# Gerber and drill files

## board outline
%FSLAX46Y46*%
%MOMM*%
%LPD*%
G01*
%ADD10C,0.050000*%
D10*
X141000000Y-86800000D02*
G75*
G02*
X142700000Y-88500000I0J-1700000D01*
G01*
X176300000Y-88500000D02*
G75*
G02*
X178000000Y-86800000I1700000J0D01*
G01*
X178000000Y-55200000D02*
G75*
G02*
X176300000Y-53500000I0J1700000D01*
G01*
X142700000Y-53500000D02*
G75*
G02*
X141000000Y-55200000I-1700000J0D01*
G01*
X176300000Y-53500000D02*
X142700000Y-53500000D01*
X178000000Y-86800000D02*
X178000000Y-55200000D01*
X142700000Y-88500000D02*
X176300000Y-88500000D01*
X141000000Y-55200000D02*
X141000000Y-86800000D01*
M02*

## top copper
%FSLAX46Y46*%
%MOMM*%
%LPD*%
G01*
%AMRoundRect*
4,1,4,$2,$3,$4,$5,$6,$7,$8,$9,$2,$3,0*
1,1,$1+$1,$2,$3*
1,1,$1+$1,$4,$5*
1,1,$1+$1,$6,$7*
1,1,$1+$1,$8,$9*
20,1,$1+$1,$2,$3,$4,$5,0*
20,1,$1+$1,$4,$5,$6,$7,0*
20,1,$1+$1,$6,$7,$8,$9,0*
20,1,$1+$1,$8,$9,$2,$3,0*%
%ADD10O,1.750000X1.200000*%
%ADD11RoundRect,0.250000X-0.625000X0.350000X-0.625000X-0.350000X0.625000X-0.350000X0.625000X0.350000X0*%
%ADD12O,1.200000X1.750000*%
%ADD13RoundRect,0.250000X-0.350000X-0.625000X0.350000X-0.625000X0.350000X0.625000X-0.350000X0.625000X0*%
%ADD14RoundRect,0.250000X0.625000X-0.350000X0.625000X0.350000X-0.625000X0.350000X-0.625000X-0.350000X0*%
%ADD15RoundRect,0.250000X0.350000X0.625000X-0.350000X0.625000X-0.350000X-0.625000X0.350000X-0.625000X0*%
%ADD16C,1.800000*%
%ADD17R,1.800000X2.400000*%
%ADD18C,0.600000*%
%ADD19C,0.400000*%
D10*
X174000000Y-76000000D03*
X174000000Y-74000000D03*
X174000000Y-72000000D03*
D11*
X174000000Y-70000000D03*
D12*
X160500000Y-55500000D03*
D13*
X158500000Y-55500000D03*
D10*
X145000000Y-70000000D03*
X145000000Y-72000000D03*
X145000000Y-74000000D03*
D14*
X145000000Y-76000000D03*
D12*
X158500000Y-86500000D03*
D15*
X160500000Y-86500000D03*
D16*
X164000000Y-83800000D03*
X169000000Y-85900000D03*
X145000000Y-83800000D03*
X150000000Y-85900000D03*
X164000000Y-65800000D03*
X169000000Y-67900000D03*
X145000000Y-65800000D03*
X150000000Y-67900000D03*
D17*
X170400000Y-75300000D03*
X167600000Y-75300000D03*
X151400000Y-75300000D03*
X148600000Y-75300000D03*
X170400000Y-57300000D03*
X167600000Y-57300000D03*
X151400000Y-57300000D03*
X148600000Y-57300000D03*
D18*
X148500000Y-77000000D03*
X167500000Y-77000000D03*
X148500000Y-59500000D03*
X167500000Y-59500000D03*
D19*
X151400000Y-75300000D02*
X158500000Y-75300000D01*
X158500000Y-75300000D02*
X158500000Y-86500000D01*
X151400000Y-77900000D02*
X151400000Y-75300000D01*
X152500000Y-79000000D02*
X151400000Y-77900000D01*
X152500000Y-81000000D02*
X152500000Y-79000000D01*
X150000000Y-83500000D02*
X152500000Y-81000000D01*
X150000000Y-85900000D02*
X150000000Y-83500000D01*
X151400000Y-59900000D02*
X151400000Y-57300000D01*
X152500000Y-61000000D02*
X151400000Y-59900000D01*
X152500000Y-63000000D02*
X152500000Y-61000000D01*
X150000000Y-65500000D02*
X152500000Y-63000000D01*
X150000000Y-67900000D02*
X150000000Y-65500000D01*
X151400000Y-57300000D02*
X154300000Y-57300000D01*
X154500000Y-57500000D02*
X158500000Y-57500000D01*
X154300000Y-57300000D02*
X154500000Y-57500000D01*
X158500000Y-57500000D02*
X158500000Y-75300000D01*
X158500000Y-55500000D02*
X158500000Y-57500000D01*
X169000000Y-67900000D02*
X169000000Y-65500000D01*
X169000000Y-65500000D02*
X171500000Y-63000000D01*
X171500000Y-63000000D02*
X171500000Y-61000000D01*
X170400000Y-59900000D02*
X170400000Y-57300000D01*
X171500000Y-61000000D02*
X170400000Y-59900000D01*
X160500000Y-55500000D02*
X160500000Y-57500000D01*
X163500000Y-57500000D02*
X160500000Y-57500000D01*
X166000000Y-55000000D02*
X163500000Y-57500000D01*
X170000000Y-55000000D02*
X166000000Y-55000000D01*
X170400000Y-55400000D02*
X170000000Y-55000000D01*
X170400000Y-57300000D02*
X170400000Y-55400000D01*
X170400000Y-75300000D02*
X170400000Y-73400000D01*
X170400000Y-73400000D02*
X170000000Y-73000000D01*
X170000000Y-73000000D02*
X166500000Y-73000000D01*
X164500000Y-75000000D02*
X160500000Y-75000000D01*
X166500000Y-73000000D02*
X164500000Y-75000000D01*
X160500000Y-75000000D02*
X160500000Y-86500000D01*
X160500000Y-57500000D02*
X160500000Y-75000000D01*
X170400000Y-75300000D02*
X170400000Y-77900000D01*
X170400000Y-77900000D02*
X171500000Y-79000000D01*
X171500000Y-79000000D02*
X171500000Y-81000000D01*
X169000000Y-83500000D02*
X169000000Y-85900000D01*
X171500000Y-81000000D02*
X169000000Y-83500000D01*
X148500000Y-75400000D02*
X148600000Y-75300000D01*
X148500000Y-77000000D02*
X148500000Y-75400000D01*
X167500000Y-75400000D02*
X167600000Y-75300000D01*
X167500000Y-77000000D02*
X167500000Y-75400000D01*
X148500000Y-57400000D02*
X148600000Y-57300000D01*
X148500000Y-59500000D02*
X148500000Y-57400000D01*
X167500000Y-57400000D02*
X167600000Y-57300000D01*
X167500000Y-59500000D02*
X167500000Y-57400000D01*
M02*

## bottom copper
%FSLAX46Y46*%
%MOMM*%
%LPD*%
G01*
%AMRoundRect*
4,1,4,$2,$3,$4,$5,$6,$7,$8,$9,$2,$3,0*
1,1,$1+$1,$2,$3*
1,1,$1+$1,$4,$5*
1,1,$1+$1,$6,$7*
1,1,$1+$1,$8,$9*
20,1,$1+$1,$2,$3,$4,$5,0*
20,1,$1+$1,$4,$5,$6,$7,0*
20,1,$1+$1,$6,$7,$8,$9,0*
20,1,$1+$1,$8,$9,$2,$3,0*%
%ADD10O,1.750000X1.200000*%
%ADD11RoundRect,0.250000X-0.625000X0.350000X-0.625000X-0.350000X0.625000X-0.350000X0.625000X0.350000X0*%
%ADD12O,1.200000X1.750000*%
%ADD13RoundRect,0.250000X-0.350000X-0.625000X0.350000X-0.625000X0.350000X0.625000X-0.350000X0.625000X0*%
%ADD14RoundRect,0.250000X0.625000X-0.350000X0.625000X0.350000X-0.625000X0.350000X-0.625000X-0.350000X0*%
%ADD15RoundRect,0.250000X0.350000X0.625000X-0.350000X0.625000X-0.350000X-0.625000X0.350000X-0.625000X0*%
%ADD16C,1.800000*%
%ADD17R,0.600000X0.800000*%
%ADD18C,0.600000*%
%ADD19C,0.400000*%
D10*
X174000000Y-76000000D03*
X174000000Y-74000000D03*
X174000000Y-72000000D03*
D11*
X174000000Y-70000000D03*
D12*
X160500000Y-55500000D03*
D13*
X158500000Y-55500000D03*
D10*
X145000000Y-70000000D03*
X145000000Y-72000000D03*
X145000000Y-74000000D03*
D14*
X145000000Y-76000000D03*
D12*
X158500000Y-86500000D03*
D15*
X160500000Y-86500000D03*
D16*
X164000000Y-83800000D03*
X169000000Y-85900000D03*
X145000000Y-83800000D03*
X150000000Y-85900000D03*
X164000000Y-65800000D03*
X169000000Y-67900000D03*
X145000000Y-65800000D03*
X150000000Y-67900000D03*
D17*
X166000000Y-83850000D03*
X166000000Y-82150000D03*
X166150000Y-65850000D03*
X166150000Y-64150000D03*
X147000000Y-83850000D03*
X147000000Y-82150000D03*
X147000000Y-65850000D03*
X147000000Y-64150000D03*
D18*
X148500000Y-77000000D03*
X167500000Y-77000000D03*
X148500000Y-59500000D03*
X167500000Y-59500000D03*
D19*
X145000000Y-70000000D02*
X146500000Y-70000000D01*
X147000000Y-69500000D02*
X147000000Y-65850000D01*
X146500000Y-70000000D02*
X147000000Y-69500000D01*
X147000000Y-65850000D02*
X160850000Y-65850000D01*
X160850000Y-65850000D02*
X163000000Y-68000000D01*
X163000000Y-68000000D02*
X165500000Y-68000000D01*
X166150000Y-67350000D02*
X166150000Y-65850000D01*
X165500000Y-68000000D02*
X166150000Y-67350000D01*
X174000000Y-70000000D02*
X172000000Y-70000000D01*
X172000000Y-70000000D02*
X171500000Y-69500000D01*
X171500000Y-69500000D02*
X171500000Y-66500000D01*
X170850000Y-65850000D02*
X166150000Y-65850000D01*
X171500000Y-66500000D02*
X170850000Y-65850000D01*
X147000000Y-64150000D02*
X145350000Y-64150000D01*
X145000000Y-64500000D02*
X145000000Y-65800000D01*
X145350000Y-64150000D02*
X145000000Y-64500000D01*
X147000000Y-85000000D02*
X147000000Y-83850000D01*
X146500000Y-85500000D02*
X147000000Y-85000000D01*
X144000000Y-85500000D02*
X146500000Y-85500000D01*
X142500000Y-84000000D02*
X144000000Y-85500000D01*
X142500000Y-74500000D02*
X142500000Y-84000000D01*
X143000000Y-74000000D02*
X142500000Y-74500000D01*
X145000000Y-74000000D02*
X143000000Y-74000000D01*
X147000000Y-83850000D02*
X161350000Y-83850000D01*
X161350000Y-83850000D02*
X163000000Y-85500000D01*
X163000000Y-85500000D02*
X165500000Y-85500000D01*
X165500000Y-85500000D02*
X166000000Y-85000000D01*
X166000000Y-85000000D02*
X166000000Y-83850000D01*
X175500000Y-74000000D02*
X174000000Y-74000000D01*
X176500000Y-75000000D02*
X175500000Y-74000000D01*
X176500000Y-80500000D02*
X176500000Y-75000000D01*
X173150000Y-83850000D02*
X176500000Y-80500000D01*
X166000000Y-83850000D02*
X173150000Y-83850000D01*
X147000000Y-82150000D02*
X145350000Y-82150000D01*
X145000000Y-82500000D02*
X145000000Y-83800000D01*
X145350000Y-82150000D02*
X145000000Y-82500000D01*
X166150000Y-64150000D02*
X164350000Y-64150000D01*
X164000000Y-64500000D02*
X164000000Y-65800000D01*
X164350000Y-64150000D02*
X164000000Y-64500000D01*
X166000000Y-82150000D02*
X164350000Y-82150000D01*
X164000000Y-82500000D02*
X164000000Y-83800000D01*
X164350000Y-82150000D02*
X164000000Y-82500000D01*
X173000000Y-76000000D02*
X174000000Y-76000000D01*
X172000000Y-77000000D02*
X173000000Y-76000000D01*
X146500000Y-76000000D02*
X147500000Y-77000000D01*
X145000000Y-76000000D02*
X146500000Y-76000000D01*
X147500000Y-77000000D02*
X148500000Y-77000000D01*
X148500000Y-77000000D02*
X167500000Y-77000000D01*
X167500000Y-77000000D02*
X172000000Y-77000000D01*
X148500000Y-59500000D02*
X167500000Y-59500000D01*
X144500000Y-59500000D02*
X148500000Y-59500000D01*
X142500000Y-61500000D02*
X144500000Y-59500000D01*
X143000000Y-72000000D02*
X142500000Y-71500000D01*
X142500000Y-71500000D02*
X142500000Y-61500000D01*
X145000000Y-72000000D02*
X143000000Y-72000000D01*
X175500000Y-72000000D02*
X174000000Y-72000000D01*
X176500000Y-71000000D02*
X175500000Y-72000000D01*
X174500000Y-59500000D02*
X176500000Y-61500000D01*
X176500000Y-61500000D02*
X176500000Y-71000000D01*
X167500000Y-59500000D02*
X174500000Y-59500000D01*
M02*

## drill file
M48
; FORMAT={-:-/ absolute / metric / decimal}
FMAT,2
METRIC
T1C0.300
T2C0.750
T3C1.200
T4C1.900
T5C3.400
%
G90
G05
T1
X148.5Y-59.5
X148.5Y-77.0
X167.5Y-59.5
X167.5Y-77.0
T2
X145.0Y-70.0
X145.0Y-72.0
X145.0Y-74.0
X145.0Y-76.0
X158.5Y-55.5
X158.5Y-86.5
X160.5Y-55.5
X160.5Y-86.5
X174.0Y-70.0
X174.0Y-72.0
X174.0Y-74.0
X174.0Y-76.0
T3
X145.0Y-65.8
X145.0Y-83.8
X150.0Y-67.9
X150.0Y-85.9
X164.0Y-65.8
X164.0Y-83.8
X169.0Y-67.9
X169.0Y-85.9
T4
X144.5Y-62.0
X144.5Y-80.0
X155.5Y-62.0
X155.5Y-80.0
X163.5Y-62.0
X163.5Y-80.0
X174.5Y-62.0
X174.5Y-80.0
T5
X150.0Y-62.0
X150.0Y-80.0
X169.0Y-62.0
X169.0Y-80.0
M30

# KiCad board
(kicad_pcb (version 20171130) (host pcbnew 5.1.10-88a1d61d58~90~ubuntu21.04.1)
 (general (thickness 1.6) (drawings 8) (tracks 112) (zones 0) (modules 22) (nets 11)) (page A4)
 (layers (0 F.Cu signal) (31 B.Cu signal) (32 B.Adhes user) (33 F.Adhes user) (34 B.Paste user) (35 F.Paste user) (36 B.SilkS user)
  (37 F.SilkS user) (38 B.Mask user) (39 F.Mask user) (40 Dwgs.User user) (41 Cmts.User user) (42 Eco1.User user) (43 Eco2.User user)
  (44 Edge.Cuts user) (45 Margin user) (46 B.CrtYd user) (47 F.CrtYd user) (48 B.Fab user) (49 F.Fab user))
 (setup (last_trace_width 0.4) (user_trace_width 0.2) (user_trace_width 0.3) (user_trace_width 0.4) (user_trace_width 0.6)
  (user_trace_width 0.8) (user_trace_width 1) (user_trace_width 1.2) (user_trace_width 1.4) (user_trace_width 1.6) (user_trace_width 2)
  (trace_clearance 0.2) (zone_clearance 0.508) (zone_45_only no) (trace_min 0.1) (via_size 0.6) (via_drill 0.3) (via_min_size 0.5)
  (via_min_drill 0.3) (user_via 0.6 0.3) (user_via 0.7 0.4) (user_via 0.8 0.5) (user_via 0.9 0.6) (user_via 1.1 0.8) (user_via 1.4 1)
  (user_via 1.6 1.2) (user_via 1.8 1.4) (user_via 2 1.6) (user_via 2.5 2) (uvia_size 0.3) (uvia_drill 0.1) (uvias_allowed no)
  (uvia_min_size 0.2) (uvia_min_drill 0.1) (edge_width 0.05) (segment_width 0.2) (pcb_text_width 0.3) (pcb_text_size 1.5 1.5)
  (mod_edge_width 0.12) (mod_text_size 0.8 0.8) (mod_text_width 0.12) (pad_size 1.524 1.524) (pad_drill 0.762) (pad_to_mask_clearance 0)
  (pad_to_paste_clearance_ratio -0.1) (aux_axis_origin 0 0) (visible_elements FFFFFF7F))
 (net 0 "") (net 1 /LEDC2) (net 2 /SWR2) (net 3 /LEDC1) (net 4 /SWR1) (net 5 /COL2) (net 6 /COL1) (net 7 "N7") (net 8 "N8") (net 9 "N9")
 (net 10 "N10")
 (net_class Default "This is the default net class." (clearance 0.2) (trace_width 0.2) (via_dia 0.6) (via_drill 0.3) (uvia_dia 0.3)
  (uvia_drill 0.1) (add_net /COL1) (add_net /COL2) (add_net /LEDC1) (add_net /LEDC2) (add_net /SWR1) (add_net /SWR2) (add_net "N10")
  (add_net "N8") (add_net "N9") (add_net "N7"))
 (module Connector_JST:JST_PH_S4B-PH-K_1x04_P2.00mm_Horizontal (layer B.Cu) (at 174 70 270)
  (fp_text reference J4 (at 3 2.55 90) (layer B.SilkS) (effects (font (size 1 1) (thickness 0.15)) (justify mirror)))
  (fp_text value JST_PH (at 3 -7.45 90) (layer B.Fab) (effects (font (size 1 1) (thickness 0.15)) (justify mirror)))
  (pad 4 thru_hole oval (at 6 0 270) (size 1.2 1.75) (drill 0.75) (layers *.Cu *.Mask) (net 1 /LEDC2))
  (pad 3 thru_hole oval (at 4 0 270) (size 1.2 1.75) (drill 0.75) (layers *.Cu *.Mask) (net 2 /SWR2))
  (pad 2 thru_hole oval (at 2 0 270) (size 1.2 1.75) (drill 0.75) (layers *.Cu *.Mask) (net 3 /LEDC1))
  (pad 1 thru_hole roundrect (at 0 0 270) (size 1.2 1.75) (drill 0.75) (layers *.Cu *.Mask) (roundrect_rratio 0.208333) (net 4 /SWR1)))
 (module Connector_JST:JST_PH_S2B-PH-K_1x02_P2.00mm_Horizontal (layer B.Cu) (at 158.5 55.5)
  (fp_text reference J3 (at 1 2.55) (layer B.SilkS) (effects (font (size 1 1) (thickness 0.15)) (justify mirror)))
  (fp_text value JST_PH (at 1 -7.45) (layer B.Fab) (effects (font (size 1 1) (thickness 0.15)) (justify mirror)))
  (pad 2 thru_hole oval (at 2 0) (size 1.2 1.75) (drill 0.75) (layers *.Cu *.Mask) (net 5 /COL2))
  (pad 1 thru_hole roundrect (at 0 0) (size 1.2 1.75) (drill 0.75) (layers *.Cu *.Mask) (roundrect_rratio 0.208333) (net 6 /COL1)))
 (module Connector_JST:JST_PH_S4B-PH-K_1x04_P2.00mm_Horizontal (layer B.Cu) (at 145 76 90)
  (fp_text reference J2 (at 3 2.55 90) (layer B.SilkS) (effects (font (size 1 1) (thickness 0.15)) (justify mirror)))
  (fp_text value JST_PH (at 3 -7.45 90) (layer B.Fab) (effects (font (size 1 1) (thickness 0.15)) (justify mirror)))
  (pad 4 thru_hole oval (at 6 0 90) (size 1.2 1.75) (drill 0.75) (layers *.Cu *.Mask) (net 4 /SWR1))
  (pad 3 thru_hole oval (at 4 0 90) (size 1.2 1.75) (drill 0.75) (layers *.Cu *.Mask) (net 3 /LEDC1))
  (pad 2 thru_hole oval (at 2 0 90) (size 1.2 1.75) (drill 0.75) (layers *.Cu *.Mask) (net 2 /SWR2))
  (pad 1 thru_hole roundrect (at 0 0 90) (size 1.2 1.75) (drill 0.75) (layers *.Cu *.Mask) (roundrect_rratio 0.208333) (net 1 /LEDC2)))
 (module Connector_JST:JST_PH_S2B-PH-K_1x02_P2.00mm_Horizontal (layer B.Cu) (at 160.5 86.5 180)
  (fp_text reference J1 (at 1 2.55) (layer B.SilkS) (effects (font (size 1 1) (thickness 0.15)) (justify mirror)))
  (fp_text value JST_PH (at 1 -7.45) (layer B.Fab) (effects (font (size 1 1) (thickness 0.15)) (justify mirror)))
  (pad 2 thru_hole oval (at 2 0 180) (size 1.2 1.75) (drill 0.75) (layers *.Cu *.Mask) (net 6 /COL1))
  (pad 1 thru_hole roundrect (at 0 0 180) (size 1.2 1.75) (drill 0.75) (layers *.Cu *.Mask) (roundrect_rratio 0.208333) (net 5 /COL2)))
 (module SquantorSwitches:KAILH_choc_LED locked (layer F.Cu) (at 169 80 180)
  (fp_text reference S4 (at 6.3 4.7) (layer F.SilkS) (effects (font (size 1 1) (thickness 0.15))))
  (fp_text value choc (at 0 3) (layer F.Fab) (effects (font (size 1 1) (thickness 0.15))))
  (pad 2 thru_hole circle (at 5 -3.8 180) (size 1.8 1.8) (drill 1.2) (layers *.Cu *.Mask) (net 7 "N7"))
  (pad 1 thru_hole circle (at 0 -5.9 180) (size 1.8 1.8) (drill 1.2) (layers *.Cu *.Mask) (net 5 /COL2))
  (pad "" np_thru_hole circle (at 5.5 0 180) (size 1.9 1.9) (drill 1.9) (layers *.Cu *.Mask))
  (pad "" np_thru_hole circle (at -5.5 0 180) (size 1.9 1.9) (drill 1.9) (layers *.Cu *.Mask))
  (pad "" np_thru_hole circle (at 0 0 180) (size 3.4 3.4) (drill 3.4) (layers *.Cu *.Mask)))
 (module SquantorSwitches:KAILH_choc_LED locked (layer F.Cu) (at 150 80 180)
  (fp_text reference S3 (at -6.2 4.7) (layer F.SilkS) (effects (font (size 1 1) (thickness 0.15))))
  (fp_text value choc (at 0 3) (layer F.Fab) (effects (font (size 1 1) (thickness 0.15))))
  (pad 2 thru_hole circle (at 5 -3.8 180) (size 1.8 1.8) (drill 1.2) (layers *.Cu *.Mask) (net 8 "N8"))
  (pad 1 thru_hole circle (at 0 -5.9 180) (size 1.8 1.8) (drill 1.2) (layers *.Cu *.Mask) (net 6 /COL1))
  (pad "" np_thru_hole circle (at 5.5 0 180) (size 1.9 1.9) (drill 1.9) (layers *.Cu *.Mask))
  (pad "" np_thru_hole circle (at -5.5 0 180) (size 1.9 1.9) (drill 1.9) (layers *.Cu *.Mask))
  (pad "" np_thru_hole circle (at 0 0 180) (size 3.4 3.4) (drill 3.4) (layers *.Cu *.Mask)))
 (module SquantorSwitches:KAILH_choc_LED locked (layer F.Cu) (at 169 62 180)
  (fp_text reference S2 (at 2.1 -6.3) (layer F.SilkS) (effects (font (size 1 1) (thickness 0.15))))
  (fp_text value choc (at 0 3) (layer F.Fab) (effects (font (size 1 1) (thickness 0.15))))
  (pad 2 thru_hole circle (at 5 -3.8 180) (size 1.8 1.8) (drill 1.2) (layers *.Cu *.Mask) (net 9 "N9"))
  (pad 1 thru_hole circle (at 0 -5.9 180) (size 1.8 1.8) (drill 1.2) (layers *.Cu *.Mask) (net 5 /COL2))
  (pad "" np_thru_hole circle (at 5.5 0 180) (size 1.9 1.9) (drill 1.9) (layers *.Cu *.Mask))
  (pad "" np_thru_hole circle (at -5.5 0 180) (size 1.9 1.9) (drill 1.9) (layers *.Cu *.Mask))
  (pad "" np_thru_hole circle (at 0 0 180) (size 3.4 3.4) (drill 3.4) (layers *.Cu *.Mask)))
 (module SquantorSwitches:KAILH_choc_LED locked (layer F.Cu) (at 150 62 180)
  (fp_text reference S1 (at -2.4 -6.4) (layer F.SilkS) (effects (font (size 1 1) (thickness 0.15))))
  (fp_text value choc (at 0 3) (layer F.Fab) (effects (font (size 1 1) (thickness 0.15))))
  (pad 2 thru_hole circle (at 5 -3.8 180) (size 1.8 1.8) (drill 1.2) (layers *.Cu *.Mask) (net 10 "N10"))
  (pad 1 thru_hole circle (at 0 -5.9 180) (size 1.8 1.8) (drill 1.2) (layers *.Cu *.Mask) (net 6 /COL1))
  (pad "" np_thru_hole circle (at 5.5 0 180) (size 1.9 1.9) (drill 1.9) (layers *.Cu *.Mask))
  (pad "" np_thru_hole circle (at -5.5 0 180) (size 1.9 1.9) (drill 1.9) (layers *.Cu *.Mask))
  (pad "" np_thru_hole circle (at 0 0 180) (size 3.4 3.4) (drill 3.4) (layers *.Cu *.Mask)))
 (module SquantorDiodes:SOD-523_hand (layer B.Cu) (at 166 83 90)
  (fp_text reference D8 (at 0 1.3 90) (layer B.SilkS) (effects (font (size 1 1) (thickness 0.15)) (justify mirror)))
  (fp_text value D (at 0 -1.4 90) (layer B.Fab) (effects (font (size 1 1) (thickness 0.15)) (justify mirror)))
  (pad 1 smd rect (at -0.85 0 90) (size 0.8 0.6) (layers B.Cu B.Paste B.Mask) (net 2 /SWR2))
  (pad 2 smd rect (at 0.85 0 90) (size 0.8 0.6) (layers B.Cu B.Paste B.Mask) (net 7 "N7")))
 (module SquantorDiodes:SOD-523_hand (layer B.Cu) (at 166.15 65 90)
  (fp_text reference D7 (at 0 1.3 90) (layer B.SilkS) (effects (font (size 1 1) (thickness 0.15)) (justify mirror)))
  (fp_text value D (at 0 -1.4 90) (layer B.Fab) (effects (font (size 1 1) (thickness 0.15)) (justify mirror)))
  (pad 1 smd rect (at -0.85 0 90) (size 0.8 0.6) (layers B.Cu B.Paste B.Mask) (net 4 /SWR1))
  (pad 2 smd rect (at 0.85 0 90) (size 0.8 0.6) (layers B.Cu B.Paste B.Mask) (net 9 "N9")))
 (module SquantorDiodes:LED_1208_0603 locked (layer F.Cu) (at 169 75.3)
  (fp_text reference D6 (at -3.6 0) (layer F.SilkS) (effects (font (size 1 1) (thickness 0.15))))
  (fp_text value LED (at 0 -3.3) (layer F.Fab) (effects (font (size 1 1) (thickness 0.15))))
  (pad 2 smd rect (at 1.4 0) (size 1.8 2.4) (layers F.Cu F.Paste F.Mask) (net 5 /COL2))
  (pad 1 smd rect (at -1.4 0) (size 1.8 2.4) (layers F.Cu F.Paste F.Mask) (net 1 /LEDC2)))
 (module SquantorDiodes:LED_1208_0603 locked (layer F.Cu) (at 150 75.3)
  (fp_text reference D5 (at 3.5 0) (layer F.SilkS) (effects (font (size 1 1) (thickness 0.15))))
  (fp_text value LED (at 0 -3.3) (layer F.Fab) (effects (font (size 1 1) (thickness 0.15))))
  (pad 2 smd rect (at 1.4 0) (size 1.8 2.4) (layers F.Cu F.Paste F.Mask) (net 6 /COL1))
  (pad 1 smd rect (at -1.4 0) (size 1.8 2.4) (layers F.Cu F.Paste F.Mask) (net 1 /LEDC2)))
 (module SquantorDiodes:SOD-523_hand (layer B.Cu) (at 147 83 90)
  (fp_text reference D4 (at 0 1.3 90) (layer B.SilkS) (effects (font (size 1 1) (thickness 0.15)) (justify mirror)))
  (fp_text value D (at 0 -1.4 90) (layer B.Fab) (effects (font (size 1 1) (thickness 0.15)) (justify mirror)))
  (pad 1 smd rect (at -0.85 0 90) (size 0.8 0.6) (layers B.Cu B.Paste B.Mask) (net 2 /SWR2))
  (pad 2 smd rect (at 0.85 0 90) (size 0.8 0.6) (layers B.Cu B.Paste B.Mask) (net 8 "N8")))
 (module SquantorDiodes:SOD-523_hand (layer B.Cu) (at 147 65 90)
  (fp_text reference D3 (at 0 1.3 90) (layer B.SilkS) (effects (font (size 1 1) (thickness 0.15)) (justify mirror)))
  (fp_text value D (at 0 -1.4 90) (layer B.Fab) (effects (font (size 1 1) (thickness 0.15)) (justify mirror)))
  (pad 1 smd rect (at -0.85 0 90) (size 0.8 0.6) (layers B.Cu B.Paste B.Mask) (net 4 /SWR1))
  (pad 2 smd rect (at 0.85 0 90) (size 0.8 0.6) (layers B.Cu B.Paste B.Mask) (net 10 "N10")))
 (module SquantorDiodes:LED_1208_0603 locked (layer F.Cu) (at 169 57.3)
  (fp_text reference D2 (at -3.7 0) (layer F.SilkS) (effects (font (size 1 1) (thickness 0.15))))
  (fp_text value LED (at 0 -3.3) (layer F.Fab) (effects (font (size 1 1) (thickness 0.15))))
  (pad 2 smd rect (at 1.4 0) (size 1.8 2.4) (layers F.Cu F.Paste F.Mask) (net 5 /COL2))
  (pad 1 smd rect (at -1.4 0) (size 1.8 2.4) (layers F.Cu F.Paste F.Mask) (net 3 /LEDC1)))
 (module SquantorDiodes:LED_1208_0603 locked (layer F.Cu) (at 150 57.3)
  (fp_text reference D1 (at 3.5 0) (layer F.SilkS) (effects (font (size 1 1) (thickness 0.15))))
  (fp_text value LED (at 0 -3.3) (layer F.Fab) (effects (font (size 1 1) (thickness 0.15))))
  (pad 2 smd rect (at 1.4 0) (size 1.8 2.4) (layers F.Cu F.Paste F.Mask) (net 6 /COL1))
  (pad 1 smd rect (at -1.4 0) (size 1.8 2.4) (layers F.Cu F.Paste F.Mask) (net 3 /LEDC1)))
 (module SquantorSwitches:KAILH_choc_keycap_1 (layer F.Cu) (at 169 80)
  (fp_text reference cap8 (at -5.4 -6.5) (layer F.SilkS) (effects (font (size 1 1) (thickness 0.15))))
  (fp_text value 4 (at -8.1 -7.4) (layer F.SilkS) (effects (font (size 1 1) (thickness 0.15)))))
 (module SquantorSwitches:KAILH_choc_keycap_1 (layer F.Cu) (at 150 80)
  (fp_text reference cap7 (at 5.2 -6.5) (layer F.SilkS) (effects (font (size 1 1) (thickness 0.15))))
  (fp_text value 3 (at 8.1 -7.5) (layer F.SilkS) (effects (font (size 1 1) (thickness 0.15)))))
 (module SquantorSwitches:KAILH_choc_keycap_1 (layer F.Cu) (at 169 62)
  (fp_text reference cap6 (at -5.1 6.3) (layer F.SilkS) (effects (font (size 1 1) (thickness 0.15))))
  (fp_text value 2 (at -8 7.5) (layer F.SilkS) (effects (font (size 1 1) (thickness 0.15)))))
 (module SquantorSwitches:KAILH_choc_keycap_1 (layer F.Cu) (at 150 62)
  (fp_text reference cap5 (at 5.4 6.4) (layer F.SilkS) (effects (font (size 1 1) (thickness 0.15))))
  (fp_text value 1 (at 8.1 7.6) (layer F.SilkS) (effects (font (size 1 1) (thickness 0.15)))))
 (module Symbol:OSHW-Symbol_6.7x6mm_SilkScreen (layer B.Cu) (at 159.5 71 180)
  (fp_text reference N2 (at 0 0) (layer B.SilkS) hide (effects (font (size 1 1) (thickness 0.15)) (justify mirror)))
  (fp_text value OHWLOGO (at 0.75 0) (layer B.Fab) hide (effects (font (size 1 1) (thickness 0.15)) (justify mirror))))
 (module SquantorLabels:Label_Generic (layer B.Cu) (at 160.3 74.7 180)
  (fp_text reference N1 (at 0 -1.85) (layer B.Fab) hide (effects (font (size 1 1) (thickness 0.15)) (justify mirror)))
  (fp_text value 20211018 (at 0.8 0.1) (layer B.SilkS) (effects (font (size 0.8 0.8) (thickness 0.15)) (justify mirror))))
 (gr_arc (start 141 88.5) (end 142.7 88.5) (angle -90) (layer Edge.Cuts) (width 0.05))
 (gr_arc (start 178 88.5) (end 178 86.8) (angle -90) (layer Edge.Cuts) (width 0.05))
 (gr_arc (start 178 53.5) (end 176.3 53.5) (angle -90) (layer Edge.Cuts) (width 0.05))
 (gr_arc (start 141 53.5) (end 141 55.2) (angle -90) (layer Edge.Cuts) (width 0.05))
 (gr_line (start 176.3 53.5) (end 142.7 53.5) (layer Edge.Cuts) (width 0.05))
 (gr_line (start 178 86.8) (end 178 55.2) (layer Edge.Cuts) (width 0.05))
 (gr_line (start 142.7 88.5) (end 176.3 88.5) (layer Edge.Cuts) (width 0.05))
 (gr_line (start 141 55.2) (end 141 86.8) (layer Edge.Cuts) (width 0.05))
 (segment (start 151.4 75.3) (end 158.5 75.3) (width 0.4) (layer F.Cu) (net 6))
 (segment (start 158.5 75.3) (end 158.5 86.5) (width 0.4) (layer F.Cu) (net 6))
 (segment (start 151.4 77.9) (end 151.4 75.3) (width 0.4) (layer F.Cu) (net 6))
 (segment (start 152.5 79) (end 151.4 77.9) (width 0.4) (layer F.Cu) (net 6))
 (segment (start 152.5 81) (end 152.5 79) (width 0.4) (layer F.Cu) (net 6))
 (segment (start 150 83.5) (end 152.5 81) (width 0.4) (layer F.Cu) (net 6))
 (segment (start 150 85.9) (end 150 83.5) (width 0.4) (layer F.Cu) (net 6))
 (segment (start 151.4 59.9) (end 151.4 57.3) (width 0.4) (layer F.Cu) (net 6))
 (segment (start 152.5 61) (end 151.4 59.9) (width 0.4) (layer F.Cu) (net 6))
 (segment (start 152.5 63) (end 152.5 61) (width 0.4) (layer F.Cu) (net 6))
 (segment (start 150 65.5) (end 152.5 63) (width 0.4) (layer F.Cu) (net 6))
 (segment (start 150 67.9) (end 150 65.5) (width 0.4) (layer F.Cu) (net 6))
 (segment (start 151.4 57.3) (end 154.3 57.3) (width 0.4) (layer F.Cu) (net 6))
 (segment (start 154.5 57.5) (end 158.5 57.5) (width 0.4) (layer F.Cu) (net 6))
 (segment (start 154.3 57.3) (end 154.5 57.5) (width 0.4) (layer F.Cu) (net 6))
 (segment (start 158.5 57.5) (end 158.5 75.3) (width 0.4) (layer F.Cu) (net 6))
 (segment (start 158.5 55.5) (end 158.5 57.5) (width 0.4) (layer F.Cu) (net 6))
 (segment (start 145 70) (end 146.5 70) (width 0.4) (layer B.Cu) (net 4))
 (segment (start 147 69.5) (end 147 65.85) (width 0.4) (layer B.Cu) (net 4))
 (segment (start 146.5 70) (end 147 69.5) (width 0.4) (layer B.Cu) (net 4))
 (segment (start 147 65.85) (end 160.85 65.85) (width 0.4) (layer B.Cu) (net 4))
 (segment (start 160.85 65.85) (end 163 68) (width 0.4) (layer B.Cu) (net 4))
 (segment (start 163 68) (end 165.5 68) (width 0.4) (layer B.Cu) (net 4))
 (segment (start 166.15 67.35) (end 166.15 65.85) (width 0.4) (layer B.Cu) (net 4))
 (segment (start 165.5 68) (end 166.15 67.35) (width 0.4) (layer B.Cu) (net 4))
 (segment (start 174 70) (end 172 70) (width 0.4) (layer B.Cu) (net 4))
 (segment (start 172 70) (end 171.5 69.5) (width 0.4) (layer B.Cu) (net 4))
 (segment (start 171.5 69.5) (end 171.5 66.5) (width 0.4) (layer B.Cu) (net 4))
 (segment (start 170.85 65.85) (end 166.15 65.85) (width 0.4) (layer B.Cu) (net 4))
 (segment (start 171.5 66.5) (end 170.85 65.85) (width 0.4) (layer B.Cu) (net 4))
 (segment (start 147 64.15) (end 145.35 64.15) (width 0.4) (layer B.Cu) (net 10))
 (segment (start 145 64.5) (end 145 65.8) (width 0.4) (layer B.Cu) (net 10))
 (segment (start 145.35 64.15) (end 145 64.5) (width 0.4) (layer B.Cu) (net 10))
 (segment (start 147 85) (end 147 83.85) (width 0.4) (layer B.Cu) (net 2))
 (segment (start 146.5 85.5) (end 147 85) (width 0.4) (layer B.Cu) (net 2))
 (segment (start 144 85.5) (end 146.5 85.5) (width 0.4) (layer B.Cu) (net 2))
 (segment (start 142.5 84) (end 144 85.5) (width 0.4) (layer B.Cu) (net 2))
 (segment (start 142.5 74.5) (end 142.5 84) (width 0.4) (layer B.Cu) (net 2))
 (segment (start 143 74) (end 142.5 74.5) (width 0.4) (layer B.Cu) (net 2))
 (segment (start 145 74) (end 143 74) (width 0.4) (layer B.Cu) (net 2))
 (segment (start 147 83.85) (end 161.35 83.85) (width 0.4) (layer B.Cu) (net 2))
 (segment (start 161.35 83.85) (end 163 85.5) (width 0.4) (layer B.Cu) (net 2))
 (segment (start 163 85.5) (end 165.5 85.5) (width 0.4) (layer B.Cu) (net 2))
 (segment (start 165.5 85.5) (end 166 85) (width 0.4) (layer B.Cu) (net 2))
 (segment (start 166 85) (end 166 83.85) (width 0.4) (layer B.Cu) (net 2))
 (segment (start 175.5 74) (end 174 74) (width 0.4) (layer B.Cu) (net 2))
 (segment (start 176.5 75) (end 175.5 74) (width 0.4) (layer B.Cu) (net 2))
 (segment (start 176.5 80.5) (end 176.5 75) (width 0.4) (layer B.Cu) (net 2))
 (segment (start 173.15 83.85) (end 176.5 80.5) (width 0.4) (layer B.Cu) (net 2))
 (segment (start 166 83.85) (end 173.15 83.85) (width 0.4) (layer B.Cu) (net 2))
 (segment (start 147 82.15) (end 145.35 82.15) (width 0.4) (layer B.Cu) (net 8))
 (segment (start 145 82.5) (end 145 83.8) (width 0.4) (layer B.Cu) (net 8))
 (segment (start 145.35 82.15) (end 145 82.5) (width 0.4) (layer B.Cu) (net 8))
 (segment (start 169 67.9) (end 169 65.5) (width 0.4) (layer F.Cu) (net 5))
 (segment (start 169 65.5) (end 171.5 63) (width 0.4) (layer F.Cu) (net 5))
 (segment (start 171.5 63) (end 171.5 61) (width 0.4) (layer F.Cu) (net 5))
 (segment (start 170.4 59.9) (end 170.4 57.3) (width 0.4) (layer F.Cu) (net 5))
 (segment (start 171.5 61) (end 170.4 59.9) (width 0.4) (layer F.Cu) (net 5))
 (segment (start 160.5 55.5) (end 160.5 57.5) (width 0.4) (layer F.Cu) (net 5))
 (segment (start 163.5 57.5) (end 160.5 57.5) (width 0.4) (layer F.Cu) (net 5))
 (segment (start 166 55) (end 163.5 57.5) (width 0.4) (layer F.Cu) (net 5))
 (segment (start 170 55) (end 166 55) (width 0.4) (layer F.Cu) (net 5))
 (segment (start 170.4 55.4) (end 170 55) (width 0.4) (layer F.Cu) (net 5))
 (segment (start 170.4 57.3) (end 170.4 55.4) (width 0.4) (layer F.Cu) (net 5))
 (segment (start 170.4 75.3) (end 170.4 73.4) (width 0.4) (layer F.Cu) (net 5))
 (segment (start 170.4 73.4) (end 170 73) (width 0.4) (layer F.Cu) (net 5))
 (segment (start 170 73) (end 166.5 73) (width 0.4) (layer F.Cu) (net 5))
 (segment (start 164.5 75) (end 160.5 75) (width 0.4) (layer F.Cu) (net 5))
 (segment (start 166.5 73) (end 164.5 75) (width 0.4) (layer F.Cu) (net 5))
 (segment (start 160.5 75) (end 160.5 86.5) (width 0.4) (layer F.Cu) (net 5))
 (segment (start 160.5 57.5) (end 160.5 75) (width 0.4) (layer F.Cu) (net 5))
 (segment (start 170.4 75.3) (end 170.4 77.9) (width 0.4) (layer F.Cu) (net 5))
 (segment (start 170.4 77.9) (end 171.5 79) (width 0.4) (layer F.Cu) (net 5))
 (segment (start 171.5 79) (end 171.5 81) (width 0.4) (layer F.Cu) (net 5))
 (segment (start 169 83.5) (end 169 85.9) (width 0.4) (layer F.Cu) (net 5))
 (segment (start 171.5 81) (end 169 83.5) (width 0.4) (layer F.Cu) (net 5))
 (segment (start 166.15 64.15) (end 164.35 64.15) (width 0.4) (layer B.Cu) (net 9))
 (segment (start 164 64.5) (end 164 65.8) (width 0.4) (layer B.Cu) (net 9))
 (segment (start 164.35 64.15) (end 164 64.5) (width 0.4) (layer B.Cu) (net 9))
 (segment (start 166 82.15) (end 164.35 82.15) (width 0.4) (layer B.Cu) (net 7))
 (segment (start 164 82.5) (end 164 83.8) (width 0.4) (layer B.Cu) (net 7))
 (segment (start 164.35 82.15) (end 164 82.5) (width 0.4) (layer B.Cu) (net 7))
 (segment (start 173 76) (end 174 76) (width 0.4) (layer B.Cu) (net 1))
 (segment (start 172 77) (end 173 76) (width 0.4) (layer B.Cu) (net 1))
 (segment (start 146.5 76) (end 147.5 77) (width 0.4) (layer B.Cu) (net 1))
 (segment (start 145 76) (end 146.5 76) (width 0.4) (layer B.Cu) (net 1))
 (via (at 148.5 77) (size 0.6) (drill 0.3) (layers F.Cu B.Cu) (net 1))
 (segment (start 147.5 77) (end 148.5 77) (width 0.4) (layer B.Cu) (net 1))
 (segment (start 148.5 75.4) (end 148.6 75.3) (width 0.4) (layer F.Cu) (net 1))
 (segment (start 148.5 77) (end 148.5 75.4) (width 0.4) (layer F.Cu) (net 1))
 (via (at 167.5 77) (size 0.6) (drill 0.3) (layers F.Cu B.Cu) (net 1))
 (segment (start 148.5 77) (end 167.5 77) (width 0.4) (layer B.Cu) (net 1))
 (segment (start 167.5 77) (end 172 77) (width 0.4) (layer B.Cu) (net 1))
 (segment (start 167.5 75.4) (end 167.6 75.3) (width 0.4) (layer F.Cu) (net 1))
 (segment (start 167.5 77) (end 167.5 75.4) (width 0.4) (layer F.Cu) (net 1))
 (via (at 148.5 59.5) (size 0.6) (drill 0.3) (layers F.Cu B.Cu) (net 3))
 (segment (start 148.5 57.4) (end 148.6 57.3) (width 0.4) (layer F.Cu) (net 3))
 (segment (start 148.5 59.5) (end 148.5 57.4) (width 0.4) (layer F.Cu) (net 3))
 (via (at 167.5 59.5) (size 0.6) (drill 0.3) (layers F.Cu B.Cu) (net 3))
 (segment (start 148.5 59.5) (end 167.5 59.5) (width 0.4) (layer B.Cu) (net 3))
 (segment (start 167.5 57.4) (end 167.6 57.3) (width 0.4) (layer F.Cu) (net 3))
 (segment (start 167.5 59.5) (end 167.5 57.4) (width 0.4) (layer F.Cu) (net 3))
 (segment (start 144.5 59.5) (end 148.5 59.5) (width 0.4) (layer B.Cu) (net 3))
 (segment (start 142.5 61.5) (end 144.5 59.5) (width 0.4) (layer B.Cu) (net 3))
 (segment (start 143 72) (end 142.5 71.5) (width 0.4) (layer B.Cu) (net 3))
 (segment (start 142.5 71.5) (end 142.5 61.5) (width 0.4) (layer B.Cu) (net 3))
 (segment (start 145 72) (end 143 72) (width 0.4) (layer B.Cu) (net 3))
 (segment (start 175.5 72) (end 174 72) (width 0.4) (layer B.Cu) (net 3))
 (segment (start 176.5 71) (end 175.5 72) (width 0.4) (layer B.Cu) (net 3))
 (segment (start 174.5 59.5) (end 176.5 61.5) (width 0.4) (layer B.Cu) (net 3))
 (segment (start 176.5 61.5) (end 176.5 71) (width 0.4) (layer B.Cu) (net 3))
 (segment (start 167.5 59.5) (end 174.5 59.5) (width 0.4) (layer B.Cu) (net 3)))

